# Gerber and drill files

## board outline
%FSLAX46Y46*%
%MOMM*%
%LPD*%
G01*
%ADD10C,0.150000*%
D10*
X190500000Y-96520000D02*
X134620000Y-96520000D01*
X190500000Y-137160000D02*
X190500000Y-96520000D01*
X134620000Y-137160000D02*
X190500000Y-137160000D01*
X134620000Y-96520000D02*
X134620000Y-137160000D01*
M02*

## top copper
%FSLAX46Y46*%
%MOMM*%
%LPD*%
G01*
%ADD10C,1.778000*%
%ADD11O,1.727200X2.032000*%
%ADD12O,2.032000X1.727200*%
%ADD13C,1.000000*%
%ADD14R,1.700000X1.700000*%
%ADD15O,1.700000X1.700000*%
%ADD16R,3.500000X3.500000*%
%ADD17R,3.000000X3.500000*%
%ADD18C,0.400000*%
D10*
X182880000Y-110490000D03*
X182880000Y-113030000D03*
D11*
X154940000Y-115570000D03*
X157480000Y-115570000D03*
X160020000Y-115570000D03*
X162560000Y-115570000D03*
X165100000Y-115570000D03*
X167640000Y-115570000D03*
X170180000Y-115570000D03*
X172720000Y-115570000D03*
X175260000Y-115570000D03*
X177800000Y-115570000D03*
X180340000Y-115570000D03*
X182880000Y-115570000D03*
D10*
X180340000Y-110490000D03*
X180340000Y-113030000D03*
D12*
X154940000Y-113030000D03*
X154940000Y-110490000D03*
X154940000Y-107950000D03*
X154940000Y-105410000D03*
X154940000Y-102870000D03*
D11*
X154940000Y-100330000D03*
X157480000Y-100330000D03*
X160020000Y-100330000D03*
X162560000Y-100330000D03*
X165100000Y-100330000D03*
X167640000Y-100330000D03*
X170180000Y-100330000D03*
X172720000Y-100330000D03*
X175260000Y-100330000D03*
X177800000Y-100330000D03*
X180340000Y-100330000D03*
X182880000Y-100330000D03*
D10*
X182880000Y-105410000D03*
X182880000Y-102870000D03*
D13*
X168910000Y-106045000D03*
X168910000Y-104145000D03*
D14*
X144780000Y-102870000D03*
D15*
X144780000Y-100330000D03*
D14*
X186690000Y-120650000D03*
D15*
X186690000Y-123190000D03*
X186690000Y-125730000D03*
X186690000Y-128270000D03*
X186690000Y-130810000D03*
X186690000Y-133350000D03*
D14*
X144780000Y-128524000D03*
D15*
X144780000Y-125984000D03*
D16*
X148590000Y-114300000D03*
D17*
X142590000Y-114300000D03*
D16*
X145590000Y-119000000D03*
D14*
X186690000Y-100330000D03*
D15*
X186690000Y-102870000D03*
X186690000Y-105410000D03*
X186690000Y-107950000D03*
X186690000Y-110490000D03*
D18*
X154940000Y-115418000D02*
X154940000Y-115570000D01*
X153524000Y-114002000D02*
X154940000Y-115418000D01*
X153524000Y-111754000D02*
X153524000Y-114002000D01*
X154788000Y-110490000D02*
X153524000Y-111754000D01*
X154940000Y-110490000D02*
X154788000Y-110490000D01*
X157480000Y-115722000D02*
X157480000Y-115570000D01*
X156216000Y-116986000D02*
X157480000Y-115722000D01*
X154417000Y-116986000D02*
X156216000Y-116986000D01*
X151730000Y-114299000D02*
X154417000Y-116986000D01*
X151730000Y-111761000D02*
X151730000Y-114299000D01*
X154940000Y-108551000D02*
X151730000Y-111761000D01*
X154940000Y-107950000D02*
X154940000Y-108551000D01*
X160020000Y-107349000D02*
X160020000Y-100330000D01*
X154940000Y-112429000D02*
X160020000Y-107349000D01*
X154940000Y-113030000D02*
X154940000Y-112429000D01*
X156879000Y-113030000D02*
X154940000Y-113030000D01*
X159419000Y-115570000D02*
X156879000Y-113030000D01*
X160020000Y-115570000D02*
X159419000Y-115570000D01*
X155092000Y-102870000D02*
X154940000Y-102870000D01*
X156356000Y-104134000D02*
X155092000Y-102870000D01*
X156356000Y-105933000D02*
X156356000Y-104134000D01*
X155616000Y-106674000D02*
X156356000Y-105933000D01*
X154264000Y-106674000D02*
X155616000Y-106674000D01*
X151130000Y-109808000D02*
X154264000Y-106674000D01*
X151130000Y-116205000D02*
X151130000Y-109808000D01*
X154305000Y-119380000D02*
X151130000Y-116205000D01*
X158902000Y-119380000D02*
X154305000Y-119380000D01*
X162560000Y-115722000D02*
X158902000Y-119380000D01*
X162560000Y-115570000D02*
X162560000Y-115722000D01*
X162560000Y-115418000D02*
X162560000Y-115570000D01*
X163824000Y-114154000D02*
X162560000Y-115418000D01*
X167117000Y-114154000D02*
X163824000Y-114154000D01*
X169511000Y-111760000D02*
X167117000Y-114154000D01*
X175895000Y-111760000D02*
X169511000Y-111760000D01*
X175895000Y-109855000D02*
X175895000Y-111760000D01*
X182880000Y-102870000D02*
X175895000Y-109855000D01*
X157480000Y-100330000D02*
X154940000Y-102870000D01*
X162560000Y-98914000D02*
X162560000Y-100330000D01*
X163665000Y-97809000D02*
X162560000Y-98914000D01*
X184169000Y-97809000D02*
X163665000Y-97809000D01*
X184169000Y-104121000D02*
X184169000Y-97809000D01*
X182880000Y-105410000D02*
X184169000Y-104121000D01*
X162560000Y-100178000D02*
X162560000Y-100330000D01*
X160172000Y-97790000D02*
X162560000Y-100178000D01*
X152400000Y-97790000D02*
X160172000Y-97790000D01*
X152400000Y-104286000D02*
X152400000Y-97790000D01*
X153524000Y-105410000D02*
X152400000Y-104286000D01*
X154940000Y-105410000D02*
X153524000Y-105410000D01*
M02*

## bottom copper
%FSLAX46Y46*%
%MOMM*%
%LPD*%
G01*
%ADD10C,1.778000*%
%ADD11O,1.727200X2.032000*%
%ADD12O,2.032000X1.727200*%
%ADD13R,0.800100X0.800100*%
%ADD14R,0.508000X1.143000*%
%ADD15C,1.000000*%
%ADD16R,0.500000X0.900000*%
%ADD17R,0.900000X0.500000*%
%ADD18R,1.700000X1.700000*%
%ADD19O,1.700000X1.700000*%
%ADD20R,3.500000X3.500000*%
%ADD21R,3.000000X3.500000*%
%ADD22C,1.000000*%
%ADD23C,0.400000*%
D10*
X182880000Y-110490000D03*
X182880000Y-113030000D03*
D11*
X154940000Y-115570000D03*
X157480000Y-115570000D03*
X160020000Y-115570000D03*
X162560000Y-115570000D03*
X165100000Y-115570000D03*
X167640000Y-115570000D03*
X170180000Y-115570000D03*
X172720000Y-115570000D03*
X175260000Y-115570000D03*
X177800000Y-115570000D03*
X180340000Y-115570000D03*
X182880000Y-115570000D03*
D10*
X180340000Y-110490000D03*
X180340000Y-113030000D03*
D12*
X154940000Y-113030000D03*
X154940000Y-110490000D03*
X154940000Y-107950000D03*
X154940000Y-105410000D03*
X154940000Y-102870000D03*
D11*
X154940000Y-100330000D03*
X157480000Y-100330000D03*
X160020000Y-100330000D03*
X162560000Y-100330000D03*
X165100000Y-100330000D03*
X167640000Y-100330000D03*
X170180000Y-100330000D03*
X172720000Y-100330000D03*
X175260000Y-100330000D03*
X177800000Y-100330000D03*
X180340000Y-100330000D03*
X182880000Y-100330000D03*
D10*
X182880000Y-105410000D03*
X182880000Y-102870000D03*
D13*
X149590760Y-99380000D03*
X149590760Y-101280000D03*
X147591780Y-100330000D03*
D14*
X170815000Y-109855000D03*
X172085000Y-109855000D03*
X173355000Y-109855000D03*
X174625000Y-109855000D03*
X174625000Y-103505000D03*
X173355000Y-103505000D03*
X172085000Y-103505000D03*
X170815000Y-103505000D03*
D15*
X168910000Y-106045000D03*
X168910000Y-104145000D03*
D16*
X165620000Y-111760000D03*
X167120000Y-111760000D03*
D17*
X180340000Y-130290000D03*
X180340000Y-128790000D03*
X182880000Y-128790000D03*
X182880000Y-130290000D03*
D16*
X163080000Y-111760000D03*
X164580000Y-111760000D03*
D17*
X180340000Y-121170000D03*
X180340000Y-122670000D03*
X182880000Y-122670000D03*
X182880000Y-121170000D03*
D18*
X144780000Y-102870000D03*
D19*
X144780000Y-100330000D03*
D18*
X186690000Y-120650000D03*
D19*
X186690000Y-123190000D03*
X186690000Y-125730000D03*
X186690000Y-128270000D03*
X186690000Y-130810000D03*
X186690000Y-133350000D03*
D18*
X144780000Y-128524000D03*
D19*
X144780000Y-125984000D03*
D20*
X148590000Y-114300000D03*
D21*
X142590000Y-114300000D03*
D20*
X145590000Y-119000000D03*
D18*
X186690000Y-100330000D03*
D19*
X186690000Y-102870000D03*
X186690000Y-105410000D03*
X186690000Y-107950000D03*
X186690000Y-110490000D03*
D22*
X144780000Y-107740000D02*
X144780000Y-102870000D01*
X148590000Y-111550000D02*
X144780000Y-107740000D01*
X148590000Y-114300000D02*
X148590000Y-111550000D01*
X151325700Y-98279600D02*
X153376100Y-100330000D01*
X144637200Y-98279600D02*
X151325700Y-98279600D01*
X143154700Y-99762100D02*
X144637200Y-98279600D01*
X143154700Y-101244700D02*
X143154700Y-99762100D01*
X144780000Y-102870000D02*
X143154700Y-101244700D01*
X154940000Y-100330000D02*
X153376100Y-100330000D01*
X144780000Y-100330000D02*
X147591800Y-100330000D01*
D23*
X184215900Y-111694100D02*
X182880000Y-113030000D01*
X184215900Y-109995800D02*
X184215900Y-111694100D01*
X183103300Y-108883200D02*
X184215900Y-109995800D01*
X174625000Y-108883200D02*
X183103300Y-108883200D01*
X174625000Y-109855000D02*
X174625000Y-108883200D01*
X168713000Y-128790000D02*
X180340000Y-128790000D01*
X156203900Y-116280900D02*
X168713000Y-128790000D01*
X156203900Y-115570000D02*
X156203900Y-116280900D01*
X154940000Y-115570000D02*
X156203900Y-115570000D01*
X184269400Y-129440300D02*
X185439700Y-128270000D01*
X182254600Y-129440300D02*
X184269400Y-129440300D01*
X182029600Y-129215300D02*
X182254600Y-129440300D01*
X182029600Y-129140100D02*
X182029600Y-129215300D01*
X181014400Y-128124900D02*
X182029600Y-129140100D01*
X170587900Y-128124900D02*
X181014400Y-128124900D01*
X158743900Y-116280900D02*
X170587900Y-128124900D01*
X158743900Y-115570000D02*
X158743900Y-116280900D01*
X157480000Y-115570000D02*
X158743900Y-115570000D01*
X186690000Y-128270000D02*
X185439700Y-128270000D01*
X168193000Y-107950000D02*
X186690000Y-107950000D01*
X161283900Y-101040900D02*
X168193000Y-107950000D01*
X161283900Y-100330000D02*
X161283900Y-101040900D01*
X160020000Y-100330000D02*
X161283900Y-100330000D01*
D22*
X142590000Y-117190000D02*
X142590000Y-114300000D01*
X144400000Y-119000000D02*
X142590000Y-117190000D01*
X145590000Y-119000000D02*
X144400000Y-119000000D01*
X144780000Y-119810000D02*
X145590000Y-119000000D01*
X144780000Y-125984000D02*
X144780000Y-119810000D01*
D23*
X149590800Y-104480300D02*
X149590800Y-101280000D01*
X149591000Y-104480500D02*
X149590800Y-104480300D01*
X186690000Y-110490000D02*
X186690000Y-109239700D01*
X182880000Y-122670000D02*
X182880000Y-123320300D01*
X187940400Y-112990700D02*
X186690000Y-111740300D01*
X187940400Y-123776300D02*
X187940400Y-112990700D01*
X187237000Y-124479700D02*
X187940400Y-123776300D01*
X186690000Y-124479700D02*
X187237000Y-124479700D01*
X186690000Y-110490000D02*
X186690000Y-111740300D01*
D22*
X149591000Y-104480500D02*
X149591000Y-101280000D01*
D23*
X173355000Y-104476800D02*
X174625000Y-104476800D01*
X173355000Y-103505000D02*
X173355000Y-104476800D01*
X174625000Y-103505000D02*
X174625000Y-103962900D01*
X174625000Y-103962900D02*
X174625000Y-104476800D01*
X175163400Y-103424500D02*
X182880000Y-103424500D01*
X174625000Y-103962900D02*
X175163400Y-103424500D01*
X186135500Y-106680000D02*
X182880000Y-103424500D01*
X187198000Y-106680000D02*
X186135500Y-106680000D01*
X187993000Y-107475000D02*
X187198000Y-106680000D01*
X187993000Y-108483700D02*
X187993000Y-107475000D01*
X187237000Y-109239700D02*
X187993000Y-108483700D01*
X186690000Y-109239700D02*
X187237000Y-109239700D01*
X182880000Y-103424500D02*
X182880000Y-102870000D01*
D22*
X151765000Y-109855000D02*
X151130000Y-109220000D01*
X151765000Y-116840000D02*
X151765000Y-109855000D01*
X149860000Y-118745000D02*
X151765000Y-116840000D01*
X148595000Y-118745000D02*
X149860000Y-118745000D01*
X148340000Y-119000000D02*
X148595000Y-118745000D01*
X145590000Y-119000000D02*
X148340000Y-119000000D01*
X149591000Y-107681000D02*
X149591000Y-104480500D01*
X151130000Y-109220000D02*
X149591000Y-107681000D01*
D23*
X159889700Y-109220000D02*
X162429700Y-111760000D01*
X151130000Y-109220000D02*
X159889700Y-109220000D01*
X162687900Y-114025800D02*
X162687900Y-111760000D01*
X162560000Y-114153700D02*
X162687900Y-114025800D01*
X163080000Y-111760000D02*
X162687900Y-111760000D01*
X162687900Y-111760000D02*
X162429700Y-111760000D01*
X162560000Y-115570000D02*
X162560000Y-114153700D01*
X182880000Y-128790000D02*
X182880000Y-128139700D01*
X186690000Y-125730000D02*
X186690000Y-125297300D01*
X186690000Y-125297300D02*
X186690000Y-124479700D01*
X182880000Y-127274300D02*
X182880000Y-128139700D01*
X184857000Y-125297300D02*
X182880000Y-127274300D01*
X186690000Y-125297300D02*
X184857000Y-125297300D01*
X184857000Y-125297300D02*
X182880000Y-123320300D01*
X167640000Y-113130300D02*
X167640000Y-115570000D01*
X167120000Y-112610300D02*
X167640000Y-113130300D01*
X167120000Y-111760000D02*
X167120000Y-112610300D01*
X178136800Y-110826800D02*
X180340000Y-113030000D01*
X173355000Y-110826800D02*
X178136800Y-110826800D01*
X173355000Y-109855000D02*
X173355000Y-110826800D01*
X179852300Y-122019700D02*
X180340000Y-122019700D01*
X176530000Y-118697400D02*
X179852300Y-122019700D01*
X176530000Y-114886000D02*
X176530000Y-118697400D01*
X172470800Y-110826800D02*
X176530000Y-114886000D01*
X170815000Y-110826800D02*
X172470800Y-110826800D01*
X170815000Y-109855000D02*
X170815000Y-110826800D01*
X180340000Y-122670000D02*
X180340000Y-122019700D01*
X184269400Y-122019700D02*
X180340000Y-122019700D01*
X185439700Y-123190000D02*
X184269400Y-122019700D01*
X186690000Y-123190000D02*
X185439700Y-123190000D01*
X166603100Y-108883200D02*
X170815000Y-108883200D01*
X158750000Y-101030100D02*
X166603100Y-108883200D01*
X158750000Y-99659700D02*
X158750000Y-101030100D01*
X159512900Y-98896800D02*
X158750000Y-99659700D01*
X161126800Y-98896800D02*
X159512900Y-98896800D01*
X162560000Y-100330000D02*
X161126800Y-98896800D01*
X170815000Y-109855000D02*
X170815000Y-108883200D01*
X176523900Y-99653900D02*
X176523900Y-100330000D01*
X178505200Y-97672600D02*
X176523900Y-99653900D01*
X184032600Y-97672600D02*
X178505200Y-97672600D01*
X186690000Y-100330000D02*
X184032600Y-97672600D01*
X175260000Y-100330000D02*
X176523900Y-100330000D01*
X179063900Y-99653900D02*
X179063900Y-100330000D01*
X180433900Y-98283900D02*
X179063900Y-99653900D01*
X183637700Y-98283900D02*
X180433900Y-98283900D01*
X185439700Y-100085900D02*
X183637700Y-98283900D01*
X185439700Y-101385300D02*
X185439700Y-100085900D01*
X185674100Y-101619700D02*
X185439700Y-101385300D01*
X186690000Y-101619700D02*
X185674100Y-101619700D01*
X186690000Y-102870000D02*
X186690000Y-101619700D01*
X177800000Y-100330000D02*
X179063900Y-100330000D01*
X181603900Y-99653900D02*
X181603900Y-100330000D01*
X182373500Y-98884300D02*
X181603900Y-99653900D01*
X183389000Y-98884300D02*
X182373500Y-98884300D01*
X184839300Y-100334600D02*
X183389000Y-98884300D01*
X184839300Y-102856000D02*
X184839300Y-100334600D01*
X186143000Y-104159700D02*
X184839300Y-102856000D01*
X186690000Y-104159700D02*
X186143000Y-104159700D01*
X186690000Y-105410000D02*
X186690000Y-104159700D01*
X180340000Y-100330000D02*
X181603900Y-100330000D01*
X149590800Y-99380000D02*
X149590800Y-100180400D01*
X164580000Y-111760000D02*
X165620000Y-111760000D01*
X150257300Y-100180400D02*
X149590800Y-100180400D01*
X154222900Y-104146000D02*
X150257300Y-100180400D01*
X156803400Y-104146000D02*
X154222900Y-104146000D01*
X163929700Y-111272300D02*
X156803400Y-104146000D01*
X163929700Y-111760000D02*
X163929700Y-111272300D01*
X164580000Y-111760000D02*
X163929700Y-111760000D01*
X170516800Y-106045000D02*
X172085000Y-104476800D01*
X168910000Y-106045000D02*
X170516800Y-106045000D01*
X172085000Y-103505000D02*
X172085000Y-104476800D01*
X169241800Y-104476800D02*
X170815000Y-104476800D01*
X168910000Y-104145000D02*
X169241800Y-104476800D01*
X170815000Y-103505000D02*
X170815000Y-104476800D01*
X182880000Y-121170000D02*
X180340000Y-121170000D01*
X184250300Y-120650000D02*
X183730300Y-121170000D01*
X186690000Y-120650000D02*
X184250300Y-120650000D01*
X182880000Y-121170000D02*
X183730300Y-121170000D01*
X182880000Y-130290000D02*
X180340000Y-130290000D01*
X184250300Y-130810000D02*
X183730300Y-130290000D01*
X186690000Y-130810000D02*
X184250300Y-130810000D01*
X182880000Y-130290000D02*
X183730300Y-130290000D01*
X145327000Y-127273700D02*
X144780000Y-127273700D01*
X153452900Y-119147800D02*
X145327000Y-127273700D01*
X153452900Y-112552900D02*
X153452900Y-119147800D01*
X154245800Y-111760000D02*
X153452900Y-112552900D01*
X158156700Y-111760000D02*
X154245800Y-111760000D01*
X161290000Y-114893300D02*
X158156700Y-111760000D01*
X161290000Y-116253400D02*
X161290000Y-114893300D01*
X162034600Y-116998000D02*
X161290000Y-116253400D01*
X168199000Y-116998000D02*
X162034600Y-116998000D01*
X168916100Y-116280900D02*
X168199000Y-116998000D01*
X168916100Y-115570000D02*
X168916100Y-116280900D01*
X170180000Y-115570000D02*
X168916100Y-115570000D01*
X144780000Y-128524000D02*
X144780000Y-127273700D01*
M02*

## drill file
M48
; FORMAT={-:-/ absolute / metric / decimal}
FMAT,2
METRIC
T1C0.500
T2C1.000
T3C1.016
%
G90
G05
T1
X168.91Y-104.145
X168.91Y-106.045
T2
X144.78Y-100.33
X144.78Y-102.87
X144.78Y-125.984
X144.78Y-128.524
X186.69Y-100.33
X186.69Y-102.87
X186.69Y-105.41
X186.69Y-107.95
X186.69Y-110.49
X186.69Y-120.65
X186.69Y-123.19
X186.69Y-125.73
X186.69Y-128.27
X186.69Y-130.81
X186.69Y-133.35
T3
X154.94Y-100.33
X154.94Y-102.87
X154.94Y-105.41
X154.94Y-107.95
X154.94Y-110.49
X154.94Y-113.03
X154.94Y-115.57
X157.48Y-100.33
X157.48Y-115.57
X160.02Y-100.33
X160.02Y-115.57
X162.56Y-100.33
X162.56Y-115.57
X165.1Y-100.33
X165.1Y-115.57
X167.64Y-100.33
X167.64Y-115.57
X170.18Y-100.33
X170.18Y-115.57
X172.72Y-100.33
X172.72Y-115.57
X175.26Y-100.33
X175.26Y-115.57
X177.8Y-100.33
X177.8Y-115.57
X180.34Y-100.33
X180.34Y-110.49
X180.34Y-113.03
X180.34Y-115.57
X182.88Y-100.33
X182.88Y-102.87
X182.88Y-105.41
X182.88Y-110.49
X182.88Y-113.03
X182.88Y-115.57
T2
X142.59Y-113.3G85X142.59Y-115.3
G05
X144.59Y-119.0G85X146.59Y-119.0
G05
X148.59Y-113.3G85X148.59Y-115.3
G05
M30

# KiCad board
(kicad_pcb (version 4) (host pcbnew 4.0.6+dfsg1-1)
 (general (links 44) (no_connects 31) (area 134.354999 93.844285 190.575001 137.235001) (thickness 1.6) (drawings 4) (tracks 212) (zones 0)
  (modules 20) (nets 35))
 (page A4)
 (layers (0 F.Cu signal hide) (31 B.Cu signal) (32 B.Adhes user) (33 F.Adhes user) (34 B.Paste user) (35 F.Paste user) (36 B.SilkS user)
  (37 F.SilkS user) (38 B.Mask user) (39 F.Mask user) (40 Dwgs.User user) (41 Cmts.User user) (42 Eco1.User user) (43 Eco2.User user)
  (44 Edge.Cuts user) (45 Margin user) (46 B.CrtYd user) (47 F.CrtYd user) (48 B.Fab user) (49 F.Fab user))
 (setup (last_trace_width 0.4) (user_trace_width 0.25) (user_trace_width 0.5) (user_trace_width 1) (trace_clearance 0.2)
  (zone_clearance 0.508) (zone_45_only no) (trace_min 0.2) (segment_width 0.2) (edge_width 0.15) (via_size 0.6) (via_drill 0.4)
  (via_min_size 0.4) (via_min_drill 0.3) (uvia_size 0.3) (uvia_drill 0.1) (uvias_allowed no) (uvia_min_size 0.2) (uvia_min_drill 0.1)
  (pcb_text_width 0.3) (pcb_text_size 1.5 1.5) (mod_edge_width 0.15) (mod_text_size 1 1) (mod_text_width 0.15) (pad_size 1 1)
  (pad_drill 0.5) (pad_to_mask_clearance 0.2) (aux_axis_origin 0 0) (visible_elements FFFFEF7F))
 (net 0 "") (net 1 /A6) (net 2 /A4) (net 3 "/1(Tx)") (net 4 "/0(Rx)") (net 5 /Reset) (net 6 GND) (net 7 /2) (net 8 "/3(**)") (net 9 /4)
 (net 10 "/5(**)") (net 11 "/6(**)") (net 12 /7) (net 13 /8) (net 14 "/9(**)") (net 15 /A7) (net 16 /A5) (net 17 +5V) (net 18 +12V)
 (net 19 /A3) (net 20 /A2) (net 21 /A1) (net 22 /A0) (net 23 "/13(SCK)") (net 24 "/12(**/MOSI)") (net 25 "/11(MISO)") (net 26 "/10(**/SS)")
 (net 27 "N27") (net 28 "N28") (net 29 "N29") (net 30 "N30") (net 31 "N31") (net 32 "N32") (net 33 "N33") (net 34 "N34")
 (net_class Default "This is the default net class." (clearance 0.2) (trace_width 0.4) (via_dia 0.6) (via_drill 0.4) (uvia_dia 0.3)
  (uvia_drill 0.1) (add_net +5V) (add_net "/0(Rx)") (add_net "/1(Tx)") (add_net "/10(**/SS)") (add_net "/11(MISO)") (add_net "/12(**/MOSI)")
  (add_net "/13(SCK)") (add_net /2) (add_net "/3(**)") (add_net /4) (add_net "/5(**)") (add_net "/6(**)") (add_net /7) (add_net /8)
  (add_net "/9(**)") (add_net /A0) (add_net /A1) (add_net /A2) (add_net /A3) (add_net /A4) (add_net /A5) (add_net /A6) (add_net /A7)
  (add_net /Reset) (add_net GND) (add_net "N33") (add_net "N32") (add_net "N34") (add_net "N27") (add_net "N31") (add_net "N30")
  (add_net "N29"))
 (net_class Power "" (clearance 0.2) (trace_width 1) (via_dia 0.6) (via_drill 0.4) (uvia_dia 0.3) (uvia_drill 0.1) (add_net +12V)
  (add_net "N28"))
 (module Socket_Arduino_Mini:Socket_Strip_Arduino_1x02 (layer F.Cu) (at 182.88 110.49 270)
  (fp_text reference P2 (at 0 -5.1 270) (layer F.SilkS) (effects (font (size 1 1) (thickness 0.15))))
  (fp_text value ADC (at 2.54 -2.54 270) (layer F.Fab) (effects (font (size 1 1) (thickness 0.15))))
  (pad 1 thru_hole circle (at 0 0 270) (size 1.778 1.778) (drill 1.016) (layers *.Cu *.Mask F.SilkS) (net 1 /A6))
  (pad 2 thru_hole circle (at 2.54 0 270) (size 1.778 1.778) (drill 1.016) (layers *.Cu *.Mask F.SilkS) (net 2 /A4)))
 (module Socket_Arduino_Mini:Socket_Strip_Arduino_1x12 (layer F.Cu) (at 154.94 115.57)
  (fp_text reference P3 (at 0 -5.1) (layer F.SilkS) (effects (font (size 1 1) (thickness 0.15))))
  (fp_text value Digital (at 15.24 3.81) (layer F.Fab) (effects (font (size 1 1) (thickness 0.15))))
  (pad 1 thru_hole oval (at 0 0) (size 1.7272 2.032) (drill 1.016) (layers *.Cu *.Mask F.SilkS) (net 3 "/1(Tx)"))
  (pad 2 thru_hole oval (at 2.54 0) (size 1.7272 2.032) (drill 1.016) (layers *.Cu *.Mask F.SilkS) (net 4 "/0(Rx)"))
  (pad 3 thru_hole oval (at 5.08 0) (size 1.7272 2.032) (drill 1.016) (layers *.Cu *.Mask F.SilkS) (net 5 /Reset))
  (pad 4 thru_hole oval (at 7.62 0) (size 1.7272 2.032) (drill 1.016) (layers *.Cu *.Mask F.SilkS) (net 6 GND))
  (pad 5 thru_hole oval (at 10.16 0) (size 1.7272 2.032) (drill 1.016) (layers *.Cu *.Mask F.SilkS) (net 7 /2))
  (pad 6 thru_hole oval (at 12.7 0) (size 1.7272 2.032) (drill 1.016) (layers *.Cu *.Mask F.SilkS) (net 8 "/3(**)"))
  (pad 7 thru_hole oval (at 15.24 0) (size 1.7272 2.032) (drill 1.016) (layers *.Cu *.Mask F.SilkS) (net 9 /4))
  (pad 8 thru_hole oval (at 17.78 0) (size 1.7272 2.032) (drill 1.016) (layers *.Cu *.Mask F.SilkS) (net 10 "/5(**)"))
  (pad 9 thru_hole oval (at 20.32 0) (size 1.7272 2.032) (drill 1.016) (layers *.Cu *.Mask F.SilkS) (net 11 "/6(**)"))
  (pad 10 thru_hole oval (at 22.86 0) (size 1.7272 2.032) (drill 1.016) (layers *.Cu *.Mask F.SilkS) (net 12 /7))
  (pad 11 thru_hole oval (at 25.4 0) (size 1.7272 2.032) (drill 1.016) (layers *.Cu *.Mask F.SilkS) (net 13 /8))
  (pad 12 thru_hole oval (at 27.94 0) (size 1.7272 2.032) (drill 1.016) (layers *.Cu *.Mask F.SilkS) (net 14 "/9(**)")))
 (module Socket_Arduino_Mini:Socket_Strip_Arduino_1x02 (layer F.Cu) (at 180.34 110.49 270)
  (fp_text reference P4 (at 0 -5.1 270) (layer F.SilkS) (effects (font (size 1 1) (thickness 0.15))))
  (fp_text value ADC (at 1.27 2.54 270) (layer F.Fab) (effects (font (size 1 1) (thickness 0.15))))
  (pad 1 thru_hole circle (at 0 0 270) (size 1.778 1.778) (drill 1.016) (layers *.Cu *.Mask F.SilkS) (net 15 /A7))
  (pad 2 thru_hole circle (at 2.54 0 270) (size 1.778 1.778) (drill 1.016) (layers *.Cu *.Mask F.SilkS) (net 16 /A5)))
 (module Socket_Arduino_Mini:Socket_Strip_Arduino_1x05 (layer F.Cu) (at 154.94 113.03 90)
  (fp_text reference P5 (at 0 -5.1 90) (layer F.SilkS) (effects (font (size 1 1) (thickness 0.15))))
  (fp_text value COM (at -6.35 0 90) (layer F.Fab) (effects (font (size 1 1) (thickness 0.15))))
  (pad 1 thru_hole oval (at 0 0 90) (size 1.7272 2.032) (drill 1.016) (layers *.Cu *.Mask F.SilkS) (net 5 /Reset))
  (pad 2 thru_hole oval (at 2.54 0 90) (size 1.7272 2.032) (drill 1.016) (layers *.Cu *.Mask F.SilkS) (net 3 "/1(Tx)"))
  (pad 3 thru_hole oval (at 5.08 0 90) (size 1.7272 2.032) (drill 1.016) (layers *.Cu *.Mask F.SilkS) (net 4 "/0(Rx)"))
  (pad 4 thru_hole oval (at 7.62 0 90) (size 1.7272 2.032) (drill 1.016) (layers *.Cu *.Mask F.SilkS) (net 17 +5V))
  (pad 5 thru_hole oval (at 10.16 0 90) (size 1.7272 2.032) (drill 1.016) (layers *.Cu *.Mask F.SilkS) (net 6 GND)))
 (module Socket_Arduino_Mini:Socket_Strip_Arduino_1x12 (layer F.Cu) (at 154.94 100.33)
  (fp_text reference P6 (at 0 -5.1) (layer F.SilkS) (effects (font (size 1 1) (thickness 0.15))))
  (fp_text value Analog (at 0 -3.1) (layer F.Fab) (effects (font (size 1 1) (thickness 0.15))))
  (pad 1 thru_hole oval (at 0 0) (size 1.7272 2.032) (drill 1.016) (layers *.Cu *.Mask F.SilkS) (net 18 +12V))
  (pad 2 thru_hole oval (at 2.54 0) (size 1.7272 2.032) (drill 1.016) (layers *.Cu *.Mask F.SilkS) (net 6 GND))
  (pad 3 thru_hole oval (at 5.08 0) (size 1.7272 2.032) (drill 1.016) (layers *.Cu *.Mask F.SilkS) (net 5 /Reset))
  (pad 4 thru_hole oval (at 7.62 0) (size 1.7272 2.032) (drill 1.016) (layers *.Cu *.Mask F.SilkS) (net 17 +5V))
  (pad 5 thru_hole oval (at 10.16 0) (size 1.7272 2.032) (drill 1.016) (layers *.Cu *.Mask F.SilkS) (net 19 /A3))
  (pad 6 thru_hole oval (at 12.7 0) (size 1.7272 2.032) (drill 1.016) (layers *.Cu *.Mask F.SilkS) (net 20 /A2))
  (pad 7 thru_hole oval (at 15.24 0) (size 1.7272 2.032) (drill 1.016) (layers *.Cu *.Mask F.SilkS) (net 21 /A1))
  (pad 8 thru_hole oval (at 17.78 0) (size 1.7272 2.032) (drill 1.016) (layers *.Cu *.Mask F.SilkS) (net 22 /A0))
  (pad 9 thru_hole oval (at 20.32 0) (size 1.7272 2.032) (drill 1.016) (layers *.Cu *.Mask F.SilkS) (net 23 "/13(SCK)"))
  (pad 10 thru_hole oval (at 22.86 0) (size 1.7272 2.032) (drill 1.016) (layers *.Cu *.Mask F.SilkS) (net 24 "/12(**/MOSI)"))
  (pad 11 thru_hole oval (at 25.4 0) (size 1.7272 2.032) (drill 1.016) (layers *.Cu *.Mask F.SilkS) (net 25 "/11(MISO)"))
  (pad 12 thru_hole oval (at 27.94 0) (size 1.7272 2.032) (drill 1.016) (layers *.Cu *.Mask F.SilkS) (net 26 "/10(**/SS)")))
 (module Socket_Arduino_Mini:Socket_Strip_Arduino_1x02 (layer F.Cu) (at 182.88 105.41 90)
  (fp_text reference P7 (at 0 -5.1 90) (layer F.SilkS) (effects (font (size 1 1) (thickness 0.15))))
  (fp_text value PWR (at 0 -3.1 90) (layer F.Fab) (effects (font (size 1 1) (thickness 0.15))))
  (pad 1 thru_hole circle (at 0 0 90) (size 1.778 1.778) (drill 1.016) (layers *.Cu *.Mask F.SilkS) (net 17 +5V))
  (pad 2 thru_hole circle (at 2.54 0 90) (size 1.778 1.778) (drill 1.016) (layers *.Cu *.Mask F.SilkS) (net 6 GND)))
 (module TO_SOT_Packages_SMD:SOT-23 (layer B.Cu) (at 148.59 100.33 270)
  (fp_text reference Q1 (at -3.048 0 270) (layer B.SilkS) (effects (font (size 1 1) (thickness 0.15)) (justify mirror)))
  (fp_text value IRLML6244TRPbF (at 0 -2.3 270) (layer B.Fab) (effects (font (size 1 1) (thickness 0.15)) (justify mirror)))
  (pad 1 smd rect (at -0.95 -1.00076 270) (size 0.8001 0.8001) (layers B.Cu B.Paste B.Mask) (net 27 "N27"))
  (pad 2 smd rect (at 0.95 -1.00076 270) (size 0.8001 0.8001) (layers B.Cu B.Paste B.Mask) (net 6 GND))
  (pad 3 smd rect (at 0 0.99822 270) (size 0.8001 0.8001) (layers B.Cu B.Paste B.Mask) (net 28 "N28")))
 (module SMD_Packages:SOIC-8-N (layer B.Cu) (at 172.72 106.68)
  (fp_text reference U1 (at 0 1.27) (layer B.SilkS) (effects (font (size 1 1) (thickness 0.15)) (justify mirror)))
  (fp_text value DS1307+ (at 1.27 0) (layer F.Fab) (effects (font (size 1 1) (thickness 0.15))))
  (pad 8 smd rect (at -1.905 3.175) (size 0.508 1.143) (layers B.Cu B.Paste B.Mask) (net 17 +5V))
  (pad 7 smd rect (at -0.635 3.175) (size 0.508 1.143) (layers B.Cu B.Paste B.Mask) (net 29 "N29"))
  (pad 6 smd rect (at 0.635 3.175) (size 0.508 1.143) (layers B.Cu B.Paste B.Mask) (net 16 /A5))
  (pad 5 smd rect (at 1.905 3.175) (size 0.508 1.143) (layers B.Cu B.Paste B.Mask) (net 2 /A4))
  (pad 4 smd rect (at 1.905 -3.175) (size 0.508 1.143) (layers B.Cu B.Paste B.Mask) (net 6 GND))
  (pad 3 smd rect (at 0.635 -3.175) (size 0.508 1.143) (layers B.Cu B.Paste B.Mask) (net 6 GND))
  (pad 2 smd rect (at -0.635 -3.175) (size 0.508 1.143) (layers B.Cu B.Paste B.Mask) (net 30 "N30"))
  (pad 1 smd rect (at -1.905 -3.175) (size 0.508 1.143) (layers B.Cu B.Paste B.Mask) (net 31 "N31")))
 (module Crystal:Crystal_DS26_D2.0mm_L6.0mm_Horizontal (layer B.Cu) (at 168.91 106.045 90)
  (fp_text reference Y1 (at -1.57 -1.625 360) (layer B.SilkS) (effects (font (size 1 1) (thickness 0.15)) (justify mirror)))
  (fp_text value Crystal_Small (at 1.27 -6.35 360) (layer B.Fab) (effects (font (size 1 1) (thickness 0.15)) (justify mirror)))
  (pad 1 thru_hole circle (at 0 0 90) (size 1 1) (drill 0.5) (layers *.Cu *.Mask) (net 30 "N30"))
  (pad 2 thru_hole circle (at 1.9 0 90) (size 1 1) (drill 0.5) (layers *.Cu *.Mask) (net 31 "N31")))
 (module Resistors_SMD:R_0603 (layer B.Cu) (at 166.37 111.76)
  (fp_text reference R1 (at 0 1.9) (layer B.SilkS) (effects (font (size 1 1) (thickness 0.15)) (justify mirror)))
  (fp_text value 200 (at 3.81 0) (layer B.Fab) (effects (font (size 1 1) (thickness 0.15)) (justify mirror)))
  (pad 1 smd rect (at -0.75 0) (size 0.5 0.9) (layers B.Cu B.Paste B.Mask) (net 27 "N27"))
  (pad 2 smd rect (at 0.75 0) (size 0.5 0.9) (layers B.Cu B.Paste B.Mask) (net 8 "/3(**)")))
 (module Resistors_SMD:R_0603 (layer B.Cu) (at 180.34 129.54 90)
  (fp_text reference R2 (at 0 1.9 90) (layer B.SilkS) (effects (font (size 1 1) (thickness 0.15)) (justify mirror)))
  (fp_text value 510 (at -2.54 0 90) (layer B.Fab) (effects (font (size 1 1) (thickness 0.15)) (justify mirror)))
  (pad 1 smd rect (at -0.75 0 90) (size 0.5 0.9) (layers B.Cu B.Paste B.Mask) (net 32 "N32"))
  (pad 2 smd rect (at 0.75 0 90) (size 0.5 0.9) (layers B.Cu B.Paste B.Mask) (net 3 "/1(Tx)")))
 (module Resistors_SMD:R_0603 (layer B.Cu) (at 182.88 129.54 270)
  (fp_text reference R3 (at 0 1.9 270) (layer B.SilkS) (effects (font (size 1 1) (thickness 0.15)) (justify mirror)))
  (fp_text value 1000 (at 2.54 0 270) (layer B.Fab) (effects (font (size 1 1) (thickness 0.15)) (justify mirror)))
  (pad 1 smd rect (at -0.75 0 270) (size 0.5 0.9) (layers B.Cu B.Paste B.Mask) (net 6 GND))
  (pad 2 smd rect (at 0.75 0 270) (size 0.5 0.9) (layers B.Cu B.Paste B.Mask) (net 32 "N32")))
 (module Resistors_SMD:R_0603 (layer B.Cu) (at 163.83 111.76)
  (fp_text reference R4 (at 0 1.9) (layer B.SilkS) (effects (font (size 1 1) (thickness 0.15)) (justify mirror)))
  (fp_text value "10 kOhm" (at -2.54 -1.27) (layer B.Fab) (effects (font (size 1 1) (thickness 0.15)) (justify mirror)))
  (pad 1 smd rect (at -0.75 0) (size 0.5 0.9) (layers B.Cu B.Paste B.Mask) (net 6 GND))
  (pad 2 smd rect (at 0.75 0) (size 0.5 0.9) (layers B.Cu B.Paste B.Mask) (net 27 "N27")))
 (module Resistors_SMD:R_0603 (layer B.Cu) (at 180.34 121.92 270)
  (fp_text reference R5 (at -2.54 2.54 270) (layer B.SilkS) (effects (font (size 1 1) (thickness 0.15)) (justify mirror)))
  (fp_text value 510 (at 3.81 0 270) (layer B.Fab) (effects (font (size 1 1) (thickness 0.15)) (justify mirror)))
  (pad 1 smd rect (at -0.75 0 270) (size 0.5 0.9) (layers B.Cu B.Paste B.Mask) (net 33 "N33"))
  (pad 2 smd rect (at 0.75 0 270) (size 0.5 0.9) (layers B.Cu B.Paste B.Mask) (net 17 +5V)))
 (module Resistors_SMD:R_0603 (layer B.Cu) (at 182.88 121.92 90)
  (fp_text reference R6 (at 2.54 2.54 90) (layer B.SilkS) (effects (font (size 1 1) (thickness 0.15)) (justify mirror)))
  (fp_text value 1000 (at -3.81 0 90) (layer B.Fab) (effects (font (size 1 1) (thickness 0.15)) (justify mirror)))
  (pad 1 smd rect (at -0.75 0 90) (size 0.5 0.9) (layers B.Cu B.Paste B.Mask) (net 6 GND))
  (pad 2 smd rect (at 0.75 0 90) (size 0.5 0.9) (layers B.Cu B.Paste B.Mask) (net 33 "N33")))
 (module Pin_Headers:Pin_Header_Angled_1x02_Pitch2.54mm (layer F.Cu) (at 144.78 102.87 180)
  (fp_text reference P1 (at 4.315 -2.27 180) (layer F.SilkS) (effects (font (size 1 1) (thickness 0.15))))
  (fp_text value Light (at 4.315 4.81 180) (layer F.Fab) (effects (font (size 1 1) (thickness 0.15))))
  (pad 1 thru_hole rect (at 0 0 180) (size 1.7 1.7) (drill 1) (layers *.Cu *.Mask) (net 18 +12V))
  (pad 2 thru_hole oval (at 0 2.54 180) (size 1.7 1.7) (drill 1) (layers *.Cu *.Mask) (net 28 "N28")))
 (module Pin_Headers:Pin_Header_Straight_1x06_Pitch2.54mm (layer F.Cu) (at 186.69 120.65)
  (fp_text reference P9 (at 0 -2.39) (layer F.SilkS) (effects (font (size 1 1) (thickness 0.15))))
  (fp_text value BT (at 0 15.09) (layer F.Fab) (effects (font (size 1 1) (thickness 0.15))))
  (pad 1 thru_hole rect (at 0 0) (size 1.7 1.7) (drill 1) (layers *.Cu *.Mask) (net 33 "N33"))
  (pad 2 thru_hole oval (at 0 2.54) (size 1.7 1.7) (drill 1) (layers *.Cu *.Mask) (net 17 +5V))
  (pad 3 thru_hole oval (at 0 5.08) (size 1.7 1.7) (drill 1) (layers *.Cu *.Mask) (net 6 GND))
  (pad 4 thru_hole oval (at 0 7.62) (size 1.7 1.7) (drill 1) (layers *.Cu *.Mask) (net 4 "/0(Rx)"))
  (pad 5 thru_hole oval (at 0 10.16) (size 1.7 1.7) (drill 1) (layers *.Cu *.Mask) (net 32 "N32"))
  (pad 6 thru_hole oval (at 0 12.7) (size 1.7 1.7) (drill 1) (layers *.Cu *.Mask) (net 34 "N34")))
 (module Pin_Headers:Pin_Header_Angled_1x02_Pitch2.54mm (layer F.Cu) (at 144.78 128.524 180)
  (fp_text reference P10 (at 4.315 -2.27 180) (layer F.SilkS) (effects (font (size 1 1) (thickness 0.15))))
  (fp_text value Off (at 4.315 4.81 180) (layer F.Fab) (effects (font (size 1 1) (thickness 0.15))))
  (pad 1 thru_hole rect (at 0 0 180) (size 1.7 1.7) (drill 1) (layers *.Cu *.Mask) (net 9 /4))
  (pad 2 thru_hole oval (at 0 2.54 180) (size 1.7 1.7) (drill 1) (layers *.Cu *.Mask) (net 6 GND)))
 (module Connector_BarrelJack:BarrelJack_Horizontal (layer F.Cu) (at 148.59 114.3)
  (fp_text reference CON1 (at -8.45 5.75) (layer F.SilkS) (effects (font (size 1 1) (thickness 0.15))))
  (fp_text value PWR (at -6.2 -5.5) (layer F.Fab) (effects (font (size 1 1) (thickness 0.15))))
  (pad 1 thru_hole rect (at 0 0) (size 3.5 3.5) (drill oval 1 3) (layers *.Cu *.Mask) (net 18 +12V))
  (pad 2 thru_hole rect (at -6 0) (size 3 3.5) (drill oval 1 3) (layers *.Cu *.Mask) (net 6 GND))
  (pad 3 thru_hole rect (at -3 4.7) (size 3.5 3.5) (drill oval 3 1) (layers *.Cu *.Mask) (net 6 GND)))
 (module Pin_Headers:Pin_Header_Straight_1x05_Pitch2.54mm (layer F.Cu) (at 186.69 100.33)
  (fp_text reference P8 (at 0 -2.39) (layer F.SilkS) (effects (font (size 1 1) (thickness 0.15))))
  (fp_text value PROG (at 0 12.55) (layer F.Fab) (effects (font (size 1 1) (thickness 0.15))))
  (pad 1 thru_hole rect (at 0 0) (size 1.7 1.7) (drill 1) (layers *.Cu *.Mask) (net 23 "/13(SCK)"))
  (pad 2 thru_hole oval (at 0 2.54) (size 1.7 1.7) (drill 1) (layers *.Cu *.Mask) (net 24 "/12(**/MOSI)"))
  (pad 3 thru_hole oval (at 0 5.08) (size 1.7 1.7) (drill 1) (layers *.Cu *.Mask) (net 25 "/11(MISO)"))
  (pad 4 thru_hole oval (at 0 7.62) (size 1.7 1.7) (drill 1) (layers *.Cu *.Mask) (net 5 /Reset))
  (pad 5 thru_hole oval (at 0 10.16) (size 1.7 1.7) (drill 1) (layers *.Cu *.Mask) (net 6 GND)))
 (gr_line (start 190.5 96.52) (end 134.62 96.52) (angle 90) (layer Edge.Cuts) (width 0.15))
 (gr_line (start 190.5 137.16) (end 190.5 96.52) (angle 90) (layer Edge.Cuts) (width 0.15))
 (gr_line (start 134.62 137.16) (end 190.5 137.16) (angle 90) (layer Edge.Cuts) (width 0.15))
 (gr_line (start 134.62 96.52) (end 134.62 137.16) (angle 90) (layer Edge.Cuts) (width 0.15))
 (segment (start 144.78 107.74) (end 144.78 102.87) (width 1) (layer B.Cu) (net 18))
 (segment (start 148.59 111.55) (end 144.78 107.74) (width 1) (layer B.Cu) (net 18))
 (segment (start 148.59 114.3) (end 148.59 111.55) (width 1) (layer B.Cu) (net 18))
 (segment (start 151.3257 98.2796) (end 153.3761 100.33) (width 1) (layer B.Cu) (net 18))
 (segment (start 144.6372 98.2796) (end 151.3257 98.2796) (width 1) (layer B.Cu) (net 18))
 (segment (start 143.1547 99.7621) (end 144.6372 98.2796) (width 1) (layer B.Cu) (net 18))
 (segment (start 143.1547 101.2447) (end 143.1547 99.7621) (width 1) (layer B.Cu) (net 18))
 (segment (start 144.78 102.87) (end 143.1547 101.2447) (width 1) (layer B.Cu) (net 18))
 (segment (start 154.94 100.33) (end 153.3761 100.33) (width 1) (layer B.Cu) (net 18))
 (segment (start 144.78 100.33) (end 147.5918 100.33) (width 1) (layer B.Cu) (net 28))
 (segment (start 184.2159 111.6941) (end 182.88 113.03) (width 0.4) (layer B.Cu) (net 2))
 (segment (start 184.2159 109.9958) (end 184.2159 111.6941) (width 0.4) (layer B.Cu) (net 2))
 (segment (start 183.1033 108.8832) (end 184.2159 109.9958) (width 0.4) (layer B.Cu) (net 2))
 (segment (start 174.625 108.8832) (end 183.1033 108.8832) (width 0.4) (layer B.Cu) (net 2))
 (segment (start 174.625 109.855) (end 174.625 108.8832) (width 0.4) (layer B.Cu) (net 2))
 (segment (start 154.94 115.418) (end 154.94 115.57) (width 0.4) (layer F.Cu) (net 3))
 (segment (start 153.524 114.002) (end 154.94 115.418) (width 0.4) (layer F.Cu) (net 3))
 (segment (start 153.524 111.754) (end 153.524 114.002) (width 0.4) (layer F.Cu) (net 3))
 (segment (start 154.788 110.49) (end 153.524 111.754) (width 0.4) (layer F.Cu) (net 3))
 (segment (start 154.94 110.49) (end 154.788 110.49) (width 0.4) (layer F.Cu) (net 3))
 (segment (start 168.713 128.79) (end 180.34 128.79) (width 0.4) (layer B.Cu) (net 3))
 (segment (start 156.2039 116.2809) (end 168.713 128.79) (width 0.4) (layer B.Cu) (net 3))
 (segment (start 156.2039 115.57) (end 156.2039 116.2809) (width 0.4) (layer B.Cu) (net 3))
 (segment (start 154.94 115.57) (end 156.2039 115.57) (width 0.4) (layer B.Cu) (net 3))
 (segment (start 157.48 115.722) (end 157.48 115.57) (width 0.4) (layer F.Cu) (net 4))
 (segment (start 156.216 116.986) (end 157.48 115.722) (width 0.4) (layer F.Cu) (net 4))
 (segment (start 154.417 116.986) (end 156.216 116.986) (width 0.4) (layer F.Cu) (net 4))
 (segment (start 151.73 114.299) (end 154.417 116.986) (width 0.4) (layer F.Cu) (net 4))
 (segment (start 151.73 111.761) (end 151.73 114.299) (width 0.4) (layer F.Cu) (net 4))
 (segment (start 154.94 108.551) (end 151.73 111.761) (width 0.4) (layer F.Cu) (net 4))
 (segment (start 154.94 107.95) (end 154.94 108.551) (width 0.4) (layer F.Cu) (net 4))
 (segment (start 184.2694 129.4403) (end 185.4397 128.27) (width 0.4) (layer B.Cu) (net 4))
 (segment (start 182.2546 129.4403) (end 184.2694 129.4403) (width 0.4) (layer B.Cu) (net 4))
 (segment (start 182.0296 129.2153) (end 182.2546 129.4403) (width 0.4) (layer B.Cu) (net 4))
 (segment (start 182.0296 129.1401) (end 182.0296 129.2153) (width 0.4) (layer B.Cu) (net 4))
 (segment (start 181.0144 128.1249) (end 182.0296 129.1401) (width 0.4) (layer B.Cu) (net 4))
 (segment (start 170.5879 128.1249) (end 181.0144 128.1249) (width 0.4) (layer B.Cu) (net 4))
 (segment (start 158.7439 116.2809) (end 170.5879 128.1249) (width 0.4) (layer B.Cu) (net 4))
 (segment (start 158.7439 115.57) (end 158.7439 116.2809) (width 0.4) (layer B.Cu) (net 4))
 (segment (start 157.48 115.57) (end 158.7439 115.57) (width 0.4) (layer B.Cu) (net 4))
 (segment (start 186.69 128.27) (end 185.4397 128.27) (width 0.4) (layer B.Cu) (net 4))
 (segment (start 160.02 107.349) (end 160.02 100.33) (width 0.4) (layer F.Cu) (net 5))
 (segment (start 154.94 112.429) (end 160.02 107.349) (width 0.4) (layer F.Cu) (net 5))
 (segment (start 154.94 113.03) (end 154.94 112.429) (width 0.4) (layer F.Cu) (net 5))
 (segment (start 156.879 113.03) (end 154.94 113.03) (width 0.4) (layer F.Cu) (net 5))
 (segment (start 159.419 115.57) (end 156.879 113.03) (width 0.4) (layer F.Cu) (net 5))
 (segment (start 160.02 115.57) (end 159.419 115.57) (width 0.4) (layer F.Cu) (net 5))
 (segment (start 168.193 107.95) (end 186.69 107.95) (width 0.4) (layer B.Cu) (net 5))
 (segment (start 161.2839 101.0409) (end 168.193 107.95) (width 0.4) (layer B.Cu) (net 5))
 (segment (start 161.2839 100.33) (end 161.2839 101.0409) (width 0.4) (layer B.Cu) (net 5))
 (segment (start 160.02 100.33) (end 161.2839 100.33) (width 0.4) (layer B.Cu) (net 5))
 (segment (start 155.092 102.87) (end 154.94 102.87) (width 0.4) (layer F.Cu) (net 6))
 (segment (start 156.356 104.134) (end 155.092 102.87) (width 0.4) (layer F.Cu) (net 6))
 (segment (start 156.356 105.933) (end 156.356 104.134) (width 0.4) (layer F.Cu) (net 6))
 (segment (start 155.616 106.674) (end 156.356 105.933) (width 0.4) (layer F.Cu) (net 6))
 (segment (start 154.264 106.674) (end 155.616 106.674) (width 0.4) (layer F.Cu) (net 6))
 (segment (start 151.13 109.808) (end 154.264 106.674) (width 0.4) (layer F.Cu) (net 6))
 (segment (start 151.13 116.205) (end 151.13 109.808) (width 0.4) (layer F.Cu) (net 6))
 (segment (start 154.305 119.38) (end 151.13 116.205) (width 0.4) (layer F.Cu) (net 6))
 (segment (start 158.902 119.38) (end 154.305 119.38) (width 0.4) (layer F.Cu) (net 6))
 (segment (start 162.56 115.722) (end 158.902 119.38) (width 0.4) (layer F.Cu) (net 6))
 (segment (start 162.56 115.57) (end 162.56 115.722) (width 0.4) (layer F.Cu) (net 6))
 (segment (start 162.56 115.418) (end 162.56 115.57) (width 0.4) (layer F.Cu) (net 6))
 (segment (start 163.824 114.154) (end 162.56 115.418) (width 0.4) (layer F.Cu) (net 6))
 (segment (start 167.117 114.154) (end 163.824 114.154) (width 0.4) (layer F.Cu) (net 6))
 (segment (start 169.511 111.76) (end 167.117 114.154) (width 0.4) (layer F.Cu) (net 6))
 (segment (start 175.895 111.76) (end 169.511 111.76) (width 0.4) (layer F.Cu) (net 6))
 (segment (start 175.895 109.855) (end 175.895 111.76) (width 0.4) (layer F.Cu) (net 6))
 (segment (start 182.88 102.87) (end 175.895 109.855) (width 0.4) (layer F.Cu) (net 6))
 (segment (start 157.48 100.33) (end 154.94 102.87) (width 0.4) (layer F.Cu) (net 6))
 (segment (start 142.59 117.19) (end 142.59 114.3) (width 1) (layer B.Cu) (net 6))
 (segment (start 144.4 119) (end 142.59 117.19) (width 1) (layer B.Cu) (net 6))
 (segment (start 145.59 119) (end 144.4 119) (width 1) (layer B.Cu) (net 6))
 (segment (start 144.78 119.81) (end 145.59 119) (width 1) (layer B.Cu) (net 6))
 (segment (start 144.78 125.984) (end 144.78 119.81) (width 1) (layer B.Cu) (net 6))
 (segment (start 149.5908 104.4803) (end 149.5908 101.28) (width 0.4) (layer B.Cu) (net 6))
 (segment (start 149.591 104.4805) (end 149.5908 104.4803) (width 0.4) (layer B.Cu) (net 6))
 (segment (start 186.69 110.49) (end 186.69 109.2397) (width 0.4) (layer B.Cu) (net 6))
 (segment (start 182.88 122.67) (end 182.88 123.3203) (width 0.4) (layer B.Cu) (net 6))
 (segment (start 187.9404 112.9907) (end 186.69 111.7403) (width 0.4) (layer B.Cu) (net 6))
 (segment (start 187.9404 123.7763) (end 187.9404 112.9907) (width 0.4) (layer B.Cu) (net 6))
 (segment (start 187.237 124.4797) (end 187.9404 123.7763) (width 0.4) (layer B.Cu) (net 6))
 (segment (start 186.69 124.4797) (end 187.237 124.4797) (width 0.4) (layer B.Cu) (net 6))
 (segment (start 186.69 110.49) (end 186.69 111.7403) (width 0.4) (layer B.Cu) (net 6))
 (segment (start 149.591 104.4805) (end 149.591 101.28) (width 1) (layer B.Cu) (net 6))
 (segment (start 173.355 104.4768) (end 174.625 104.4768) (width 0.4) (layer B.Cu) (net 6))
 (segment (start 173.355 103.505) (end 173.355 104.4768) (width 0.4) (layer B.Cu) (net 6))
 (segment (start 174.625 103.505) (end 174.625 103.9629) (width 0.4) (layer B.Cu) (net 6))
 (segment (start 174.625 103.9629) (end 174.625 104.4768) (width 0.4) (layer B.Cu) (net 6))
 (segment (start 175.1634 103.4245) (end 182.88 103.4245) (width 0.4) (layer B.Cu) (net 6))
 (segment (start 174.625 103.9629) (end 175.1634 103.4245) (width 0.4) (layer B.Cu) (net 6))
 (segment (start 186.1355 106.68) (end 182.88 103.4245) (width 0.4) (layer B.Cu) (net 6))
 (segment (start 187.198 106.68) (end 186.1355 106.68) (width 0.4) (layer B.Cu) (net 6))
 (segment (start 187.993 107.475) (end 187.198 106.68) (width 0.4) (layer B.Cu) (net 6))
 (segment (start 187.993 108.4837) (end 187.993 107.475) (width 0.4) (layer B.Cu) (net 6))
 (segment (start 187.237 109.2397) (end 187.993 108.4837) (width 0.4) (layer B.Cu) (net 6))
 (segment (start 186.69 109.2397) (end 187.237 109.2397) (width 0.4) (layer B.Cu) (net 6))
 (segment (start 182.88 103.4245) (end 182.88 102.87) (width 0.4) (layer B.Cu) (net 6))
 (segment (start 151.765 109.855) (end 151.13 109.22) (width 1) (layer B.Cu) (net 6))
 (segment (start 151.765 116.84) (end 151.765 109.855) (width 1) (layer B.Cu) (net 6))
 (segment (start 149.86 118.745) (end 151.765 116.84) (width 1) (layer B.Cu) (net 6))
 (segment (start 148.595 118.745) (end 149.86 118.745) (width 1) (layer B.Cu) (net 6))
 (segment (start 148.34 119) (end 148.595 118.745) (width 1) (layer B.Cu) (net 6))
 (segment (start 145.59 119) (end 148.34 119) (width 1) (layer B.Cu) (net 6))
 (segment (start 149.591 107.681) (end 149.591 104.4805) (width 1) (layer B.Cu) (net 6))
 (segment (start 151.13 109.22) (end 149.591 107.681) (width 1) (layer B.Cu) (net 6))
 (segment (start 159.8897 109.22) (end 162.4297 111.76) (width 0.4) (layer B.Cu) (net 6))
 (segment (start 151.13 109.22) (end 159.8897 109.22) (width 0.4) (layer B.Cu) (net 6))
 (segment (start 162.6879 114.0258) (end 162.6879 111.76) (width 0.4) (layer B.Cu) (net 6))
 (segment (start 162.56 114.1537) (end 162.6879 114.0258) (width 0.4) (layer B.Cu) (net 6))
 (segment (start 163.08 111.76) (end 162.6879 111.76) (width 0.4) (layer B.Cu) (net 6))
 (segment (start 162.6879 111.76) (end 162.4297 111.76) (width 0.4) (layer B.Cu) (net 6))
 (segment (start 162.56 115.57) (end 162.56 114.1537) (width 0.4) (layer B.Cu) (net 6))
 (segment (start 182.88 128.79) (end 182.88 128.1397) (width 0.4) (layer B.Cu) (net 6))
 (segment (start 186.69 125.73) (end 186.69 125.2973) (width 0.4) (layer B.Cu) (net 6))
 (segment (start 186.69 125.2973) (end 186.69 124.4797) (width 0.4) (layer B.Cu) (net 6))
 (segment (start 182.88 127.2743) (end 182.88 128.1397) (width 0.4) (layer B.Cu) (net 6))
 (segment (start 184.857 125.2973) (end 182.88 127.2743) (width 0.4) (layer B.Cu) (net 6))
 (segment (start 186.69 125.2973) (end 184.857 125.2973) (width 0.4) (layer B.Cu) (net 6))
 (segment (start 184.857 125.2973) (end 182.88 123.3203) (width 0.4) (layer B.Cu) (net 6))
 (segment (start 167.64 113.1303) (end 167.64 115.57) (width 0.4) (layer B.Cu) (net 8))
 (segment (start 167.12 112.6103) (end 167.64 113.1303) (width 0.4) (layer B.Cu) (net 8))
 (segment (start 167.12 111.76) (end 167.12 112.6103) (width 0.4) (layer B.Cu) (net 8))
 (segment (start 178.1368 110.8268) (end 180.34 113.03) (width 0.4) (layer B.Cu) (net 16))
 (segment (start 173.355 110.8268) (end 178.1368 110.8268) (width 0.4) (layer B.Cu) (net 16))
 (segment (start 173.355 109.855) (end 173.355 110.8268) (width 0.4) (layer B.Cu) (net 16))
 (segment (start 162.56 98.914) (end 162.56 100.33) (width 0.4) (layer F.Cu) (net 17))
 (segment (start 163.665 97.809) (end 162.56 98.914) (width 0.4) (layer F.Cu) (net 17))
 (segment (start 184.169 97.809) (end 163.665 97.809) (width 0.4) (layer F.Cu) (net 17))
 (segment (start 184.169 104.121) (end 184.169 97.809) (width 0.4) (layer F.Cu) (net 17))
 (segment (start 182.88 105.41) (end 184.169 104.121) (width 0.4) (layer F.Cu) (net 17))
 (segment (start 162.56 100.178) (end 162.56 100.33) (width 0.4) (layer F.Cu) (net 17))
 (segment (start 160.172 97.79) (end 162.56 100.178) (width 0.4) (layer F.Cu) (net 17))
 (segment (start 152.4 97.79) (end 160.172 97.79) (width 0.4) (layer F.Cu) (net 17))
 (segment (start 152.4 104.286) (end 152.4 97.79) (width 0.4) (layer F.Cu) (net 17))
 (segment (start 153.524 105.41) (end 152.4 104.286) (width 0.4) (layer F.Cu) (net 17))
 (segment (start 154.94 105.41) (end 153.524 105.41) (width 0.4) (layer F.Cu) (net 17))
 (segment (start 179.8523 122.0197) (end 180.34 122.0197) (width 0.4) (layer B.Cu) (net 17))
 (segment (start 176.53 118.6974) (end 179.8523 122.0197) (width 0.4) (layer B.Cu) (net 17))
 (segment (start 176.53 114.886) (end 176.53 118.6974) (width 0.4) (layer B.Cu) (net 17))
 (segment (start 172.4708 110.8268) (end 176.53 114.886) (width 0.4) (layer B.Cu) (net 17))
 (segment (start 170.815 110.8268) (end 172.4708 110.8268) (width 0.4) (layer B.Cu) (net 17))
 (segment (start 170.815 109.855) (end 170.815 110.8268) (width 0.4) (layer B.Cu) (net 17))
 (segment (start 180.34 122.67) (end 180.34 122.0197) (width 0.4) (layer B.Cu) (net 17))
 (segment (start 184.2694 122.0197) (end 180.34 122.0197) (width 0.4) (layer B.Cu) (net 17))
 (segment (start 185.4397 123.19) (end 184.2694 122.0197) (width 0.4) (layer B.Cu) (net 17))
 (segment (start 186.69 123.19) (end 185.4397 123.19) (width 0.4) (layer B.Cu) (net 17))
 (segment (start 166.6031 108.8832) (end 170.815 108.8832) (width 0.4) (layer B.Cu) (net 17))
 (segment (start 158.75 101.0301) (end 166.6031 108.8832) (width 0.4) (layer B.Cu) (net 17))
 (segment (start 158.75 99.6597) (end 158.75 101.0301) (width 0.4) (layer B.Cu) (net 17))
 (segment (start 159.5129 98.8968) (end 158.75 99.6597) (width 0.4) (layer B.Cu) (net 17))
 (segment (start 161.1268 98.8968) (end 159.5129 98.8968) (width 0.4) (layer B.Cu) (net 17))
 (segment (start 162.56 100.33) (end 161.1268 98.8968) (width 0.4) (layer B.Cu) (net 17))
 (segment (start 170.815 109.855) (end 170.815 108.8832) (width 0.4) (layer B.Cu) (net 17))
 (segment (start 176.5239 99.6539) (end 176.5239 100.33) (width 0.4) (layer B.Cu) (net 23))
 (segment (start 178.5052 97.6726) (end 176.5239 99.6539) (width 0.4) (layer B.Cu) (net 23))
 (segment (start 184.0326 97.6726) (end 178.5052 97.6726) (width 0.4) (layer B.Cu) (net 23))
 (segment (start 186.69 100.33) (end 184.0326 97.6726) (width 0.4) (layer B.Cu) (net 23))
 (segment (start 175.26 100.33) (end 176.5239 100.33) (width 0.4) (layer B.Cu) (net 23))
 (segment (start 179.0639 99.6539) (end 179.0639 100.33) (width 0.4) (layer B.Cu) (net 24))
 (segment (start 180.4339 98.2839) (end 179.0639 99.6539) (width 0.4) (layer B.Cu) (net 24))
 (segment (start 183.6377 98.2839) (end 180.4339 98.2839) (width 0.4) (layer B.Cu) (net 24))
 (segment (start 185.4397 100.0859) (end 183.6377 98.2839) (width 0.4) (layer B.Cu) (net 24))
 (segment (start 185.4397 101.3853) (end 185.4397 100.0859) (width 0.4) (layer B.Cu) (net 24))
 (segment (start 185.6741 101.6197) (end 185.4397 101.3853) (width 0.4) (layer B.Cu) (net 24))
 (segment (start 186.69 101.6197) (end 185.6741 101.6197) (width 0.4) (layer B.Cu) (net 24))
 (segment (start 186.69 102.87) (end 186.69 101.6197) (width 0.4) (layer B.Cu) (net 24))
 (segment (start 177.8 100.33) (end 179.0639 100.33) (width 0.4) (layer B.Cu) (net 24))
 (segment (start 181.6039 99.6539) (end 181.6039 100.33) (width 0.4) (layer B.Cu) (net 25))
 (segment (start 182.3735 98.8843) (end 181.6039 99.6539) (width 0.4) (layer B.Cu) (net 25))
 (segment (start 183.389 98.8843) (end 182.3735 98.8843) (width 0.4) (layer B.Cu) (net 25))
 (segment (start 184.8393 100.3346) (end 183.389 98.8843) (width 0.4) (layer B.Cu) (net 25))
 (segment (start 184.8393 102.856) (end 184.8393 100.3346) (width 0.4) (layer B.Cu) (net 25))
 (segment (start 186.143 104.1597) (end 184.8393 102.856) (width 0.4) (layer B.Cu) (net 25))
 (segment (start 186.69 104.1597) (end 186.143 104.1597) (width 0.4) (layer B.Cu) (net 25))
 (segment (start 186.69 105.41) (end 186.69 104.1597) (width 0.4) (layer B.Cu) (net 25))
 (segment (start 180.34 100.33) (end 181.6039 100.33) (width 0.4) (layer B.Cu) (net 25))
 (segment (start 149.5908 99.38) (end 149.5908 100.1804) (width 0.4) (layer B.Cu) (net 27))
 (segment (start 164.58 111.76) (end 165.62 111.76) (width 0.4) (layer B.Cu) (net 27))
 (segment (start 150.2573 100.1804) (end 149.5908 100.1804) (width 0.4) (layer B.Cu) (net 27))
 (segment (start 154.2229 104.146) (end 150.2573 100.1804) (width 0.4) (layer B.Cu) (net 27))
 (segment (start 156.8034 104.146) (end 154.2229 104.146) (width 0.4) (layer B.Cu) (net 27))
 (segment (start 163.9297 111.2723) (end 156.8034 104.146) (width 0.4) (layer B.Cu) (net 27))
 (segment (start 163.9297 111.76) (end 163.9297 111.2723) (width 0.4) (layer B.Cu) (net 27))
 (segment (start 164.58 111.76) (end 163.9297 111.76) (width 0.4) (layer B.Cu) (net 27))
 (segment (start 170.5168 106.045) (end 172.085 104.4768) (width 0.4) (layer B.Cu) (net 30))
 (segment (start 168.91 106.045) (end 170.5168 106.045) (width 0.4) (layer B.Cu) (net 30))
 (segment (start 172.085 103.505) (end 172.085 104.4768) (width 0.4) (layer B.Cu) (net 30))
 (segment (start 169.2418 104.4768) (end 170.815 104.4768) (width 0.4) (layer B.Cu) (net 31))
 (segment (start 168.91 104.145) (end 169.2418 104.4768) (width 0.4) (layer B.Cu) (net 31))
 (segment (start 170.815 103.505) (end 170.815 104.4768) (width 0.4) (layer B.Cu) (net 31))
 (segment (start 182.88 121.17) (end 180.34 121.17) (width 0.4) (layer B.Cu) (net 33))
 (segment (start 184.2503 120.65) (end 183.7303 121.17) (width 0.4) (layer B.Cu) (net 33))
 (segment (start 186.69 120.65) (end 184.2503 120.65) (width 0.4) (layer B.Cu) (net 33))
 (segment (start 182.88 121.17) (end 183.7303 121.17) (width 0.4) (layer B.Cu) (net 33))
 (segment (start 182.88 130.29) (end 180.34 130.29) (width 0.4) (layer B.Cu) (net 32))
 (segment (start 184.2503 130.81) (end 183.7303 130.29) (width 0.4) (layer B.Cu) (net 32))
 (segment (start 186.69 130.81) (end 184.2503 130.81) (width 0.4) (layer B.Cu) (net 32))
 (segment (start 182.88 130.29) (end 183.7303 130.29) (width 0.4) (layer B.Cu) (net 32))
 (segment (start 145.327 127.2737) (end 144.78 127.2737) (width 0.4) (layer B.Cu) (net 9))
 (segment (start 153.4529 119.1478) (end 145.327 127.2737) (width 0.4) (layer B.Cu) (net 9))
 (segment (start 153.4529 112.5529) (end 153.4529 119.1478) (width 0.4) (layer B.Cu) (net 9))
 (segment (start 154.2458 111.76) (end 153.4529 112.5529) (width 0.4) (layer B.Cu) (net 9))
 (segment (start 158.1567 111.76) (end 154.2458 111.76) (width 0.4) (layer B.Cu) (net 9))
 (segment (start 161.29 114.8933) (end 158.1567 111.76) (width 0.4) (layer B.Cu) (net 9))
 (segment (start 161.29 116.2534) (end 161.29 114.8933) (width 0.4) (layer B.Cu) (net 9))
 (segment (start 162.0346 116.998) (end 161.29 116.2534) (width 0.4) (layer B.Cu) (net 9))
 (segment (start 168.199 116.998) (end 162.0346 116.998) (width 0.4) (layer B.Cu) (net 9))
 (segment (start 168.9161 116.2809) (end 168.199 116.998) (width 0.4) (layer B.Cu) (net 9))
 (segment (start 168.9161 115.57) (end 168.9161 116.2809) (width 0.4) (layer B.Cu) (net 9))
 (segment (start 170.18 115.57) (end 168.9161 115.57) (width 0.4) (layer B.Cu) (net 9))
 (segment (start 144.78 128.524) (end 144.78 127.2737) (width 0.4) (layer B.Cu) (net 9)))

